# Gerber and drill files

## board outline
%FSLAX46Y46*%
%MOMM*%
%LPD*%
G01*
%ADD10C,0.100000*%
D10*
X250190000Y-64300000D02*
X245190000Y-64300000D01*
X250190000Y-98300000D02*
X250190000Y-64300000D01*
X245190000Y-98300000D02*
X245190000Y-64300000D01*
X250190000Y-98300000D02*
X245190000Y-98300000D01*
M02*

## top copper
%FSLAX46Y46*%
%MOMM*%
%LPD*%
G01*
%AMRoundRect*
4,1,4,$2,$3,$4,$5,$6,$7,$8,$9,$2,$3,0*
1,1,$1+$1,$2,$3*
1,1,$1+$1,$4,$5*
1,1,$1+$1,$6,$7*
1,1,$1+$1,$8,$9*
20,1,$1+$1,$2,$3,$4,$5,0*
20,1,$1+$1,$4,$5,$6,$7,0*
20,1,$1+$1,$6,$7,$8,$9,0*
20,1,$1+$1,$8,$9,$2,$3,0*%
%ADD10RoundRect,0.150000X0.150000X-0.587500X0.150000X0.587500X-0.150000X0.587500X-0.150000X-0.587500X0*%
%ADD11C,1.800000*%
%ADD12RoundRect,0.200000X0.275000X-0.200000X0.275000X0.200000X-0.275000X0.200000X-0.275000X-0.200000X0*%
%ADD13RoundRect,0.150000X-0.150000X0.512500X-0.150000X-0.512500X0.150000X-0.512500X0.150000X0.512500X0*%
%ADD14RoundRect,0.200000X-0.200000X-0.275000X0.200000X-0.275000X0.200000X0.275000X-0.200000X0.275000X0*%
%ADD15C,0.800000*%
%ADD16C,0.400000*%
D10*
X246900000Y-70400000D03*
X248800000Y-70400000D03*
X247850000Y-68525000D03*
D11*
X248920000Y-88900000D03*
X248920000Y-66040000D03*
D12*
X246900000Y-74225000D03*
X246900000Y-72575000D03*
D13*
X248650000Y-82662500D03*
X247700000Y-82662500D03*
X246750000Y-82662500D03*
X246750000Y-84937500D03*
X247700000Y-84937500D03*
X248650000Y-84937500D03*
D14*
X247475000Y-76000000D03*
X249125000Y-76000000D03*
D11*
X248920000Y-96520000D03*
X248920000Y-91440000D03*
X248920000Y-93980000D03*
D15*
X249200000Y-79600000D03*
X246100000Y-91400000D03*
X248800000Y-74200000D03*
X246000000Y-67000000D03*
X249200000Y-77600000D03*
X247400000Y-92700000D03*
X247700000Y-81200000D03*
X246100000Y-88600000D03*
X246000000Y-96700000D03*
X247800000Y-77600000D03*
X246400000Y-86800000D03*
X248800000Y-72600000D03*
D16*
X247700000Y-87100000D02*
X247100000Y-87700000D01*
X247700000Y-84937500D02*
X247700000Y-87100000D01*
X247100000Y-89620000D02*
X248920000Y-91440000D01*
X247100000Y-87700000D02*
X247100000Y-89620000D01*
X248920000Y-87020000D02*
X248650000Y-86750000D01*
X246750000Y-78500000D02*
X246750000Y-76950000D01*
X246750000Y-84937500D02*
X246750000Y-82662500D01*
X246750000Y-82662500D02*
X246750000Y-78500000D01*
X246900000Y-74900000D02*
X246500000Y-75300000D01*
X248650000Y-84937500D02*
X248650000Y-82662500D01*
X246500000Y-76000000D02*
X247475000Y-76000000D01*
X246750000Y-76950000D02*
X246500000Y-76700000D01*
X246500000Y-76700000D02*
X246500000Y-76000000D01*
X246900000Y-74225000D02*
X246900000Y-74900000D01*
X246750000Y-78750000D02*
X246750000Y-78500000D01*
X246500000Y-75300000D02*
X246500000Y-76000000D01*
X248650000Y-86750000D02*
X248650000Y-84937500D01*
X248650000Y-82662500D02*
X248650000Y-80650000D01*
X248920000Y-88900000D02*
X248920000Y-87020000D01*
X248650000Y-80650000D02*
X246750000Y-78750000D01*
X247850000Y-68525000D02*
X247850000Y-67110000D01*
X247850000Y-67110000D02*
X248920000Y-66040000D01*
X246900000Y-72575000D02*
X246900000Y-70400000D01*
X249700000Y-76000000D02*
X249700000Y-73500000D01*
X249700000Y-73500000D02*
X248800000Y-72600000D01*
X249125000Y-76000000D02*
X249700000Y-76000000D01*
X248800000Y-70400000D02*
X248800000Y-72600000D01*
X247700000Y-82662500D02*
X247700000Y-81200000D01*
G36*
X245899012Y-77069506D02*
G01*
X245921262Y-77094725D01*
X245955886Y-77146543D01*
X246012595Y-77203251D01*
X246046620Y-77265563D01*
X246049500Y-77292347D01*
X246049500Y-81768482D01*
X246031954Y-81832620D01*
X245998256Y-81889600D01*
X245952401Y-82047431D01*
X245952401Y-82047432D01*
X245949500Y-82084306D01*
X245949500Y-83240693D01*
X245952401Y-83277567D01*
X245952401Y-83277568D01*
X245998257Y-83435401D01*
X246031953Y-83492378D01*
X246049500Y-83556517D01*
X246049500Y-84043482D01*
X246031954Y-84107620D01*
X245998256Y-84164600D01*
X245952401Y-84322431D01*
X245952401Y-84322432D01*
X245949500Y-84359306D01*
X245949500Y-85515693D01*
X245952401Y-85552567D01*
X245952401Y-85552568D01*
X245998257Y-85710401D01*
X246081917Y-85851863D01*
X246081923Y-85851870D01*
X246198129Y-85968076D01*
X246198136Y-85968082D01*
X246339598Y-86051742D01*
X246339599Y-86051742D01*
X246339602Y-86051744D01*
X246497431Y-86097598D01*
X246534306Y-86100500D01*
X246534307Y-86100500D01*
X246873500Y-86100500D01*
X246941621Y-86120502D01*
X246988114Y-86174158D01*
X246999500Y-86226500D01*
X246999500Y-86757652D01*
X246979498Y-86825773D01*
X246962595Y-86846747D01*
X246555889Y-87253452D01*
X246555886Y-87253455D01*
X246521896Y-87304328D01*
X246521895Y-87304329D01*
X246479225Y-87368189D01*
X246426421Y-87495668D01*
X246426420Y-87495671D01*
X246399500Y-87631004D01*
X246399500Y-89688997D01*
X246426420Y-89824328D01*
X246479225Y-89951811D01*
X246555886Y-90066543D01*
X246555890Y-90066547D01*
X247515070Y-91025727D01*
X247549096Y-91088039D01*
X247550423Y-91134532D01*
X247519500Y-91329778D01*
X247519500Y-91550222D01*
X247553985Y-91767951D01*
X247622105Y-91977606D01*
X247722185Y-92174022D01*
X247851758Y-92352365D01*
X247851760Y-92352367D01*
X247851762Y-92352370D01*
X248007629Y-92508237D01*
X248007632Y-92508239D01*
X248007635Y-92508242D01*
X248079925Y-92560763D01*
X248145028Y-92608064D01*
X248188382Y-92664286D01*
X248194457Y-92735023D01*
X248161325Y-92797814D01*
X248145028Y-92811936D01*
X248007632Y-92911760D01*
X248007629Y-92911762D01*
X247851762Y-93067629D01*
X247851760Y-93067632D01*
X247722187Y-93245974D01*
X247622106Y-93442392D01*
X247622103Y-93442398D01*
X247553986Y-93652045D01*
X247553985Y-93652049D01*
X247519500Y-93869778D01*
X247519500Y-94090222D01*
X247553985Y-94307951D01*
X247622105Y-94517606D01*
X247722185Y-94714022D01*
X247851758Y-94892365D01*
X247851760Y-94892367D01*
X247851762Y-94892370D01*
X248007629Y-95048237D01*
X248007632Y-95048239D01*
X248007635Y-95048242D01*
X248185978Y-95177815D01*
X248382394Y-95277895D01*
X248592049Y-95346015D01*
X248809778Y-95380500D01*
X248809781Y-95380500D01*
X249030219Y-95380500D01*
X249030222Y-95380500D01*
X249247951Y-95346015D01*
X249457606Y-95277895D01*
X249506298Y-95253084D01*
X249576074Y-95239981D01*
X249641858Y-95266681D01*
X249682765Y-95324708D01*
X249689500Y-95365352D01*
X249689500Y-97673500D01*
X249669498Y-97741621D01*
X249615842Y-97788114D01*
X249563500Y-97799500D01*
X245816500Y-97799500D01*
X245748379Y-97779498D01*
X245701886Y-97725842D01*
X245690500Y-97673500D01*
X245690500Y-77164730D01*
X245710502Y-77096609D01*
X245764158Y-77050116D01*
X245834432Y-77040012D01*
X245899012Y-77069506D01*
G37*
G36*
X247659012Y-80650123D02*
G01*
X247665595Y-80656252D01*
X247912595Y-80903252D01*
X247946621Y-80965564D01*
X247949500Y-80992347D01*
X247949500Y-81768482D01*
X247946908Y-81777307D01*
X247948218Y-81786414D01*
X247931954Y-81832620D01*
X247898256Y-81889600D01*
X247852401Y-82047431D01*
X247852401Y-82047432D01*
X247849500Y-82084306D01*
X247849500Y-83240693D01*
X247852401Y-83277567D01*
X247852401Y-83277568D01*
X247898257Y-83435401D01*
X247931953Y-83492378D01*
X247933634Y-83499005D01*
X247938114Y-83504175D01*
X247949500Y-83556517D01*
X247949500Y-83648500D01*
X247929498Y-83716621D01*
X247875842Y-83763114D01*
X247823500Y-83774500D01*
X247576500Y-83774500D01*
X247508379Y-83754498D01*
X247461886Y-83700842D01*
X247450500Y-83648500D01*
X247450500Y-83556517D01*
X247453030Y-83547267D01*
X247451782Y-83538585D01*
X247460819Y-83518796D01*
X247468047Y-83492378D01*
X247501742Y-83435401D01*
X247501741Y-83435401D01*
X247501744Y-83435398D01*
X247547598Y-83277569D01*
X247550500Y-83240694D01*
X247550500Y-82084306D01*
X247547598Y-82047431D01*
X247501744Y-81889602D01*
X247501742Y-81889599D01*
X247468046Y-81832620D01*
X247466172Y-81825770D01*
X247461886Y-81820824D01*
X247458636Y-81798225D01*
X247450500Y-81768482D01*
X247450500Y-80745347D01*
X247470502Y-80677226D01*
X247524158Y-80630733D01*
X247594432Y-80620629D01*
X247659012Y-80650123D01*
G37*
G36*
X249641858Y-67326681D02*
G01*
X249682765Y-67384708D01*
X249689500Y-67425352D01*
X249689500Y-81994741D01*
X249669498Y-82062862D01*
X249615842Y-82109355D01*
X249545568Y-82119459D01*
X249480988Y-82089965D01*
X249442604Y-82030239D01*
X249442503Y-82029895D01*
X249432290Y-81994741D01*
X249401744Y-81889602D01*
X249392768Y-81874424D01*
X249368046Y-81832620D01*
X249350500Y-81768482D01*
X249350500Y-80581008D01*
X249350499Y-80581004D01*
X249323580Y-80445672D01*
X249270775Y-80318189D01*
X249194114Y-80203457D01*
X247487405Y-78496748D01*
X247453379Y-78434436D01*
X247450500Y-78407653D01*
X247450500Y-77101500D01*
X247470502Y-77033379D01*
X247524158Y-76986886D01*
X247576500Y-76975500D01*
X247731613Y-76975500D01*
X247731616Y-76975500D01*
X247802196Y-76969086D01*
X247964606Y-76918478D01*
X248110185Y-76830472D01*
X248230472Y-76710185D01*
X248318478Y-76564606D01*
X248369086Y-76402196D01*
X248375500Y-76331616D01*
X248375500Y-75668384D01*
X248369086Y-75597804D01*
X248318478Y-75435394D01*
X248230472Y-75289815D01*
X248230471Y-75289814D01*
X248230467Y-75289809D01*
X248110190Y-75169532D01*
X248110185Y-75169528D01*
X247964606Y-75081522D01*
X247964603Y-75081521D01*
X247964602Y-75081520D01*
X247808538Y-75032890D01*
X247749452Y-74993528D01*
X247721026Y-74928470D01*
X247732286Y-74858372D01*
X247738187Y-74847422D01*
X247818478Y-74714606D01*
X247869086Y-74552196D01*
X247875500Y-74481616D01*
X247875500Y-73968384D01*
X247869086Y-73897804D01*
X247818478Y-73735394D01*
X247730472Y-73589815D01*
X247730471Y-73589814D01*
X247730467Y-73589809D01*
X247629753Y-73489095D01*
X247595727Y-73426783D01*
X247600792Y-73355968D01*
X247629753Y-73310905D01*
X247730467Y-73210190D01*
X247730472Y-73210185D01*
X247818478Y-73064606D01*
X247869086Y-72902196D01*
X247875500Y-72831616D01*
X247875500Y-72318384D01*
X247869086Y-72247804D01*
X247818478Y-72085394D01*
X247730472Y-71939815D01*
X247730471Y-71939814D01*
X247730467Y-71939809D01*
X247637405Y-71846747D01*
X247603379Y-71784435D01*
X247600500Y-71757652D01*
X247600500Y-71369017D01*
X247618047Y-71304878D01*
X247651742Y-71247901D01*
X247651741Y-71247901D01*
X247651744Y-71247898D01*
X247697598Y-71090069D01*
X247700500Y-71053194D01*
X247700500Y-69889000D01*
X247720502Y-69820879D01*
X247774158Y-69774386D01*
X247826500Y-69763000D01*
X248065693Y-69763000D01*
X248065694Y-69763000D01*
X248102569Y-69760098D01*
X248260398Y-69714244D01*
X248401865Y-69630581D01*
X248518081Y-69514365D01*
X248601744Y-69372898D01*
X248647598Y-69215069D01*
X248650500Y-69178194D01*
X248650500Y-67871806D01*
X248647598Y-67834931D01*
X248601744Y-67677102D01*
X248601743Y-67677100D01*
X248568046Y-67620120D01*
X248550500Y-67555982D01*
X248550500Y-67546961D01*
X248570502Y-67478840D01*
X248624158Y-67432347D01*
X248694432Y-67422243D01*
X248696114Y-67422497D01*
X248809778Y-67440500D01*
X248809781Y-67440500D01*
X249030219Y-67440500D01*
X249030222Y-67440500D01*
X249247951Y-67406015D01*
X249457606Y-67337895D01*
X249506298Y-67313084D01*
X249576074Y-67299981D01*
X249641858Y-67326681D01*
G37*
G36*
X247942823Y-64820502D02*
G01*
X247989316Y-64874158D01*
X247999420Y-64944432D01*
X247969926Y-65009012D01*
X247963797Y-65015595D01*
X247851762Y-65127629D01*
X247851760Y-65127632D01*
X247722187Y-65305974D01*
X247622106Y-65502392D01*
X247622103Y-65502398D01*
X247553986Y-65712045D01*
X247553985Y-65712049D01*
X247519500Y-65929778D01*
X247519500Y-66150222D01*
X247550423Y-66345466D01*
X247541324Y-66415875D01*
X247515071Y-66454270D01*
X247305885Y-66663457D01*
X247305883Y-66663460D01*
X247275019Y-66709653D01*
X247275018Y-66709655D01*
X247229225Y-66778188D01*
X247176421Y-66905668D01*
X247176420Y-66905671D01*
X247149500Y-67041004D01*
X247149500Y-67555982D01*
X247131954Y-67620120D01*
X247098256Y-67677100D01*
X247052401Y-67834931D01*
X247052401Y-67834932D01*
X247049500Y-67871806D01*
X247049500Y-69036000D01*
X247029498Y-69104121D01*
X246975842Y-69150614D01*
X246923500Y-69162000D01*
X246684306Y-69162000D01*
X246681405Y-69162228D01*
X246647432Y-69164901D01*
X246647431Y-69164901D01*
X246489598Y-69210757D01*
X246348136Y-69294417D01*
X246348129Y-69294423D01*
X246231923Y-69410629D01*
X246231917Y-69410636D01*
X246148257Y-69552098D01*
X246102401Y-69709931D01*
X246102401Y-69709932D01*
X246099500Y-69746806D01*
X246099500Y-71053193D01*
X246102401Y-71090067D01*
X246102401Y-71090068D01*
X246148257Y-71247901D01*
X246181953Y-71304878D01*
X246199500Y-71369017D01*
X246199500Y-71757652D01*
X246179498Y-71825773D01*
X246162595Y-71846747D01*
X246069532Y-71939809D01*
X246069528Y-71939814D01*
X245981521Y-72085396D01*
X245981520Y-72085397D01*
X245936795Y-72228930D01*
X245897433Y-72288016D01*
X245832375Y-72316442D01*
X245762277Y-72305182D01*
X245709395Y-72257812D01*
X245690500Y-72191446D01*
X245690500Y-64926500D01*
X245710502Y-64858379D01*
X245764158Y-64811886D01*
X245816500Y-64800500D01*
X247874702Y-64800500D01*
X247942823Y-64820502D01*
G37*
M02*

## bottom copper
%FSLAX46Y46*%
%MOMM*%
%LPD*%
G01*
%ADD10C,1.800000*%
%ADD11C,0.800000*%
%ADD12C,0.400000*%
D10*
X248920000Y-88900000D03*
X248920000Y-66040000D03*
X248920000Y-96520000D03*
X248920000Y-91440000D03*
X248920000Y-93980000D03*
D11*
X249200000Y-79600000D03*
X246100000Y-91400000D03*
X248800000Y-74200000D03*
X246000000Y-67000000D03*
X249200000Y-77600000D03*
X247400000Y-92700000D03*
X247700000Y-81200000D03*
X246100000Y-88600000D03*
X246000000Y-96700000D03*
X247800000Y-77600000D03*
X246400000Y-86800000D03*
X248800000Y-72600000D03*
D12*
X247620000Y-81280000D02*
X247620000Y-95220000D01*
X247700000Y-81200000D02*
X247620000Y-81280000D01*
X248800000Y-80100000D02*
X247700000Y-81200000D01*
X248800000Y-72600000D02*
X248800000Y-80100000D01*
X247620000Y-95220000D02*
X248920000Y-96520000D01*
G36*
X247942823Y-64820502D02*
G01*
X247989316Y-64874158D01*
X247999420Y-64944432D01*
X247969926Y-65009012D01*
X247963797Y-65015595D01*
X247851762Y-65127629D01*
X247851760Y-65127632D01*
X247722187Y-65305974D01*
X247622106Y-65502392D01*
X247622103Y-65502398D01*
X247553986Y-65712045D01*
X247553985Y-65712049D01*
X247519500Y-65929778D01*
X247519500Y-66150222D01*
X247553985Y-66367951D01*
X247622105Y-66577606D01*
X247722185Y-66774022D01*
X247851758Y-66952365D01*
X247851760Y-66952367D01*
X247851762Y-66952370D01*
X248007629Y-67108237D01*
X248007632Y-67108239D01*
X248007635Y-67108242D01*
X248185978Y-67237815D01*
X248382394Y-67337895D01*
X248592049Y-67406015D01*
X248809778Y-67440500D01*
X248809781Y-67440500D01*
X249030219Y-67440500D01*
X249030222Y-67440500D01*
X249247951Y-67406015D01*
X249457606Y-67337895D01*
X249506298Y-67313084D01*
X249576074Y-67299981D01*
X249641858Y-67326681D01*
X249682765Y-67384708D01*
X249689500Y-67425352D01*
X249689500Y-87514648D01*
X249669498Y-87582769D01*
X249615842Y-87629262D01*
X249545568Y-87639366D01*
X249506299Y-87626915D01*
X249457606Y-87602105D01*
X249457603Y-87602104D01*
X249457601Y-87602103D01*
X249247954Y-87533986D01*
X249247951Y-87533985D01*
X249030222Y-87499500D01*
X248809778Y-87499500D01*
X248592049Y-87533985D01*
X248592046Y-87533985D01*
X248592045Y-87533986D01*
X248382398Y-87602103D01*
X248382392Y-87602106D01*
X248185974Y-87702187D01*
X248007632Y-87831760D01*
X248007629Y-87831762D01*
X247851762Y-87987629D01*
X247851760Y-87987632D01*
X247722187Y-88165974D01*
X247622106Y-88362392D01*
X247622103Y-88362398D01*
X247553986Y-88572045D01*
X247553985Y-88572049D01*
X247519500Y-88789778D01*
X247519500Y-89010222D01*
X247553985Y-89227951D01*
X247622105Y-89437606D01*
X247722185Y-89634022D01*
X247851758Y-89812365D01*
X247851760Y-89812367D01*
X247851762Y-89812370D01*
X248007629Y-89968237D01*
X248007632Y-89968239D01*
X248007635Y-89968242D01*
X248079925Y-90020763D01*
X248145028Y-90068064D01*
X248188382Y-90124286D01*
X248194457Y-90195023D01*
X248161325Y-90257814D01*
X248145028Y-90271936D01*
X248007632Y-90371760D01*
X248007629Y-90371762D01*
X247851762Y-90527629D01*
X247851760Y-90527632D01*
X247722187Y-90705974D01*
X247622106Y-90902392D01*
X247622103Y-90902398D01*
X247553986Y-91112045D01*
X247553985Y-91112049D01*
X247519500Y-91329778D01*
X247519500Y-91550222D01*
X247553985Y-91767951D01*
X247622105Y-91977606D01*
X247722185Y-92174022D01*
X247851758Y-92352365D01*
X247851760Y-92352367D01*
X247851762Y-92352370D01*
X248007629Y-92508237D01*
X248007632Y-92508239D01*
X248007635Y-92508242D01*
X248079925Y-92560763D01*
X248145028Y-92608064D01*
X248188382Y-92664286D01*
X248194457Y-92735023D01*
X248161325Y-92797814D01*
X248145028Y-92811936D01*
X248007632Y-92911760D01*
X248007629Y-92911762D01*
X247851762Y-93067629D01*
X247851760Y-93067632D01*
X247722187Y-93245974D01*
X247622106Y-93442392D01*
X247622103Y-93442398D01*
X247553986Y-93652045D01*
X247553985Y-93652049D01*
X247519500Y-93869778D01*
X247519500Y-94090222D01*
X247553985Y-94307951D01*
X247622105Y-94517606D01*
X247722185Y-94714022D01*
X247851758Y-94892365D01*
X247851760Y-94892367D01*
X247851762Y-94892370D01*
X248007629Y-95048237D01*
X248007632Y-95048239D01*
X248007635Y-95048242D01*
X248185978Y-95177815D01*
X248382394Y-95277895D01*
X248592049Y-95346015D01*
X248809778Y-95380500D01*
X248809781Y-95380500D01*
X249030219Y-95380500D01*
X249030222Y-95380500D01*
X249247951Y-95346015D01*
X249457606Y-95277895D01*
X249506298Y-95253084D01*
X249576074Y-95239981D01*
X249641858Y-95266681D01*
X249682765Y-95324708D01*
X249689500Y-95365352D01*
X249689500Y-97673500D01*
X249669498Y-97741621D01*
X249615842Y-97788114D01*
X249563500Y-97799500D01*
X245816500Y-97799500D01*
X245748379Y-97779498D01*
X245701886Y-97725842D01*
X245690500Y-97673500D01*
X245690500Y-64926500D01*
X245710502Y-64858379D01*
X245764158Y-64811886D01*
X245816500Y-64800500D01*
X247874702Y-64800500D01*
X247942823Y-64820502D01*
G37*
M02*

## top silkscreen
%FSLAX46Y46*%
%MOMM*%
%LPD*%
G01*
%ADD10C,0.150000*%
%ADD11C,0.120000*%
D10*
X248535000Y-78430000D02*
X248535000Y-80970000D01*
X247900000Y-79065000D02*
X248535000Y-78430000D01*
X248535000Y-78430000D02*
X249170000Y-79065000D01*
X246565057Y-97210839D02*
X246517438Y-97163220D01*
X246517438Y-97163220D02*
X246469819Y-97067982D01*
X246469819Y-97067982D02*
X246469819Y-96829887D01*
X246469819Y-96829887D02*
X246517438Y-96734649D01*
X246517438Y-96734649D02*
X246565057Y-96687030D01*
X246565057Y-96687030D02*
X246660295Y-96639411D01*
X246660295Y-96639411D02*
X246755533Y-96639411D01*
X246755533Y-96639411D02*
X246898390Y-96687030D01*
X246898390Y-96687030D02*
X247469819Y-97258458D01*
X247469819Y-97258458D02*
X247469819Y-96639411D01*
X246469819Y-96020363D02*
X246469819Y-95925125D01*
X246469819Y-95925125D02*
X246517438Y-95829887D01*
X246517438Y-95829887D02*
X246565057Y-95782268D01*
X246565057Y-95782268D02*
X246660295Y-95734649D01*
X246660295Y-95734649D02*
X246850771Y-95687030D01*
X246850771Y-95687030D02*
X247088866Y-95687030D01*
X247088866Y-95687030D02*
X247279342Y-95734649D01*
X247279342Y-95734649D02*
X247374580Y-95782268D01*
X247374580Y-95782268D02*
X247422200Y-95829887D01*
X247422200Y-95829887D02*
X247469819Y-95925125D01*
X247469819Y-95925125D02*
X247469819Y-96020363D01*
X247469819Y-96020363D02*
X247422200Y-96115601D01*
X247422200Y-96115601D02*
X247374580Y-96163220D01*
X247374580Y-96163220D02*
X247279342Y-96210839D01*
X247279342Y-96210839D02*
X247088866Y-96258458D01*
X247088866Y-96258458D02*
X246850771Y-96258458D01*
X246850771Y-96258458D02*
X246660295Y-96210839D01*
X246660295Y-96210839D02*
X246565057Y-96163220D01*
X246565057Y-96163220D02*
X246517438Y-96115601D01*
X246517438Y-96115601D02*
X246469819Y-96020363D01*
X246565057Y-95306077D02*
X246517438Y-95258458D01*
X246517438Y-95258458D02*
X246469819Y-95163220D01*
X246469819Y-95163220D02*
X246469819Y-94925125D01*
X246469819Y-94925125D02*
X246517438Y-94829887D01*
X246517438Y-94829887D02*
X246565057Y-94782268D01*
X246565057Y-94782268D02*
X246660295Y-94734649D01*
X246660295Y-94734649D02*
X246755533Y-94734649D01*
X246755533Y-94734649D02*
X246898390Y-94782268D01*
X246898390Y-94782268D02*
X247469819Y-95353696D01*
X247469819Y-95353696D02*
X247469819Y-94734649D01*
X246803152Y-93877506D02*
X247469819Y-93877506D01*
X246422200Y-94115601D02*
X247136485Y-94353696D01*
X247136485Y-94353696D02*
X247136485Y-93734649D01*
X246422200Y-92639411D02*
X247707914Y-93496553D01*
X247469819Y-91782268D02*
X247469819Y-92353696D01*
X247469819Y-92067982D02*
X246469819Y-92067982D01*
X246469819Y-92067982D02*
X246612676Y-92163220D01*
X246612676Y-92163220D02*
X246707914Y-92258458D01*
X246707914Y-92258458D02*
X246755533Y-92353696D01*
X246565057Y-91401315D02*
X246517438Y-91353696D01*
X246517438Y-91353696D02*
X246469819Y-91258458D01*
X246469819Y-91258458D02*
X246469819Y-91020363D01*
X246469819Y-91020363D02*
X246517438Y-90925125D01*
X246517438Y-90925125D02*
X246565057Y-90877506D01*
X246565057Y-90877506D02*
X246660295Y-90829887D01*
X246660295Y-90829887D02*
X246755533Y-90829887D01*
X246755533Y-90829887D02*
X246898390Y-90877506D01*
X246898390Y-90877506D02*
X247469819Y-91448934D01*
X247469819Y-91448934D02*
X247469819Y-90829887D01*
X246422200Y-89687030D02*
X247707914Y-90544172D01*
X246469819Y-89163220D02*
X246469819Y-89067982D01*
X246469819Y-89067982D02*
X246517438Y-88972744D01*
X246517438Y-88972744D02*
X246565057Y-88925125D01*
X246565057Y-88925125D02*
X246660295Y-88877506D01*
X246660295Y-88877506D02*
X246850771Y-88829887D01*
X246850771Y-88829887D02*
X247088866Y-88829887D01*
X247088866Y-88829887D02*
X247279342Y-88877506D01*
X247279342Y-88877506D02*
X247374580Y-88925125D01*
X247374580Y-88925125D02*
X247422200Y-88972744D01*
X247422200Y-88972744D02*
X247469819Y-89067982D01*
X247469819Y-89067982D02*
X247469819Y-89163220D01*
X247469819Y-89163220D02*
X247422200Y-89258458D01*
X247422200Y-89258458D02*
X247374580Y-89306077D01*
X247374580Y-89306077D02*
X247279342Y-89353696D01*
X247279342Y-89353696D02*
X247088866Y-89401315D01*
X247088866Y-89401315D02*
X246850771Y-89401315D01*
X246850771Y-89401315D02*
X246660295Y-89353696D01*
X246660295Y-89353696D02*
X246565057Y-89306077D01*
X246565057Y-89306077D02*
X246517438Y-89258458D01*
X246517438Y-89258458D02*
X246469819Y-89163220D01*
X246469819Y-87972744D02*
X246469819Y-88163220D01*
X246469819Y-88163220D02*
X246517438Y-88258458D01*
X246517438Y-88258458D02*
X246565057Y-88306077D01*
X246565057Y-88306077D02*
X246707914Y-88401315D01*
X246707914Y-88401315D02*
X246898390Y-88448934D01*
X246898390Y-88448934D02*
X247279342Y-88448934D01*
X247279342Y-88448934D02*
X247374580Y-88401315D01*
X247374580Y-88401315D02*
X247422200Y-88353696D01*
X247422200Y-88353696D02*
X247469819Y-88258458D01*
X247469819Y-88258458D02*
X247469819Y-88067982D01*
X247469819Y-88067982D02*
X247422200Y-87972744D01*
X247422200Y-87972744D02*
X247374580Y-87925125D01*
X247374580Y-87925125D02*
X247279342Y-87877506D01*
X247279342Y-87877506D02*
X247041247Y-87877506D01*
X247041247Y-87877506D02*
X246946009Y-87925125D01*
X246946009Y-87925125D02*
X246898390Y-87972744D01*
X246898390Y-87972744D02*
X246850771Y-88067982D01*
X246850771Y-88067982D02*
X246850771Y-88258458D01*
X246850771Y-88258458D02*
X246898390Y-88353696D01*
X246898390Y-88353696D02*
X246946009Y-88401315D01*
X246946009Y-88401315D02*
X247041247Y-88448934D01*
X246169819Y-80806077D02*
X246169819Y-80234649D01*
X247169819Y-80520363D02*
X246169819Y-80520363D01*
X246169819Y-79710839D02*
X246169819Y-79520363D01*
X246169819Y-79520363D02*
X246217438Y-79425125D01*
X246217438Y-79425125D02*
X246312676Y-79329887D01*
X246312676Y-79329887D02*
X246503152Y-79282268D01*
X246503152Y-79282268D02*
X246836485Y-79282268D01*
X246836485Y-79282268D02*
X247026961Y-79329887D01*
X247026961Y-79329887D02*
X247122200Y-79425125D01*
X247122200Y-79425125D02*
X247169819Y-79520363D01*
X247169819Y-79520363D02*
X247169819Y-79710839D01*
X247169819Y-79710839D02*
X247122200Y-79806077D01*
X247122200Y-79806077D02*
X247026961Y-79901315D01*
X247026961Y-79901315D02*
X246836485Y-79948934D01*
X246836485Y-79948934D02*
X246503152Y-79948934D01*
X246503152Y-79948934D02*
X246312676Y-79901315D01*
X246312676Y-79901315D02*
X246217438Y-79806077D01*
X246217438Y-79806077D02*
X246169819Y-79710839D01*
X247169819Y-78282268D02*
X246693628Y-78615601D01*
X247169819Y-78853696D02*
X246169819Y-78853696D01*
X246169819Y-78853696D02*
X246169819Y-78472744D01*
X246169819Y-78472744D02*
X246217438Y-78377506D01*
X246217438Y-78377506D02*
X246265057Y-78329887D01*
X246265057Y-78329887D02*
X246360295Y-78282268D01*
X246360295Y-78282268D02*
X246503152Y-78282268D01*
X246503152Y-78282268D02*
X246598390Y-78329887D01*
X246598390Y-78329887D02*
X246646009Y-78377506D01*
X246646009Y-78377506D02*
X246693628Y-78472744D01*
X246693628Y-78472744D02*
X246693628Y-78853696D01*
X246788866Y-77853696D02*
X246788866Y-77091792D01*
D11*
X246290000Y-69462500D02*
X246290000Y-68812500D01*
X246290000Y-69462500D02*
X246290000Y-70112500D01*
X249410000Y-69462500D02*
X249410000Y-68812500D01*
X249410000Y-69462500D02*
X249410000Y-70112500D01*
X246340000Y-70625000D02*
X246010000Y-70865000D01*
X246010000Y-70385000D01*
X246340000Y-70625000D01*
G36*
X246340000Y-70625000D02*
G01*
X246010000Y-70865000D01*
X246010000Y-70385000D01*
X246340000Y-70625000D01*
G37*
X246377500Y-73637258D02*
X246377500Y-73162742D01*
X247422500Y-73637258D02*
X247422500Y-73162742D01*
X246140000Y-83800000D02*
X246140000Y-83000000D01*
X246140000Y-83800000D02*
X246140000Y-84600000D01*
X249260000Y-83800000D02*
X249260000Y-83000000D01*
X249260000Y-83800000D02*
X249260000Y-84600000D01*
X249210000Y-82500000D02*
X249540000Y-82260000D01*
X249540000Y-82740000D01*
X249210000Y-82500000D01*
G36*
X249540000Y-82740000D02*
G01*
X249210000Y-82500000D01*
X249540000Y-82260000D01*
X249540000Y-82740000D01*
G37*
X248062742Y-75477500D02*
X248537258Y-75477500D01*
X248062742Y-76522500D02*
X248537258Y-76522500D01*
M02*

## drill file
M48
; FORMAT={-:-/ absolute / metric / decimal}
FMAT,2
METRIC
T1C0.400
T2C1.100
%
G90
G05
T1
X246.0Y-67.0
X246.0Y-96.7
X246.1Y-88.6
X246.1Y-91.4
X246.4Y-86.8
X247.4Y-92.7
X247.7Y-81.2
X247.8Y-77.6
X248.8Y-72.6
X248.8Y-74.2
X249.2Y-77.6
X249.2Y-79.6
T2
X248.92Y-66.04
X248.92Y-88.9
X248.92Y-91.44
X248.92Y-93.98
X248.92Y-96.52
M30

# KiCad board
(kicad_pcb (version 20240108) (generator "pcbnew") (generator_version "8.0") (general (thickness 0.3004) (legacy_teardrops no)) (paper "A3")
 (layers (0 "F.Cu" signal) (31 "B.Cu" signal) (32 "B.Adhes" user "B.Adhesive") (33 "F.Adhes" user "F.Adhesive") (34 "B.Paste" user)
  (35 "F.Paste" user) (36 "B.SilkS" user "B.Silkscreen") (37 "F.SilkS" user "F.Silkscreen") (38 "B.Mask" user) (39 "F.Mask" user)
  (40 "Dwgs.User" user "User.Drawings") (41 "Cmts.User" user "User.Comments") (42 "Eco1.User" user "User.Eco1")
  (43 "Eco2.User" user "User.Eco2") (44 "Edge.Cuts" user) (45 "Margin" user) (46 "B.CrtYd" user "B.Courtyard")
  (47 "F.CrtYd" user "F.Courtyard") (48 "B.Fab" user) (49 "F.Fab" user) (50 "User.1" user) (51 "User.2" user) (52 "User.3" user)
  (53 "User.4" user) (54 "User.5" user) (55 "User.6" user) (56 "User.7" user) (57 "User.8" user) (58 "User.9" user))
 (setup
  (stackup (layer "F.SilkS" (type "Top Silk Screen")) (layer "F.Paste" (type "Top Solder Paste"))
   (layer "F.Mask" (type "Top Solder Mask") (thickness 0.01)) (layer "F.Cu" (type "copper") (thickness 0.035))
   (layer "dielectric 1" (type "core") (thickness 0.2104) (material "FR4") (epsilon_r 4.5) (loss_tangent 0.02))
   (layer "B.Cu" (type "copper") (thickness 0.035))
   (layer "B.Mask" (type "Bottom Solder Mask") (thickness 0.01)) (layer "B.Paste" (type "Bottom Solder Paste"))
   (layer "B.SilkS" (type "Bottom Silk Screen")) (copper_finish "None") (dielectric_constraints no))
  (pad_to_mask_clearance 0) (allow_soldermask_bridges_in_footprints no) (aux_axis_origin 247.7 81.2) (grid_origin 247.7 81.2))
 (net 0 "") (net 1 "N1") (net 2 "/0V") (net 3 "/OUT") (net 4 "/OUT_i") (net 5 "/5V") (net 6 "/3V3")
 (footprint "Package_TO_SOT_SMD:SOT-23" (layer "F.Cu") (at 247.85 69.4625 90)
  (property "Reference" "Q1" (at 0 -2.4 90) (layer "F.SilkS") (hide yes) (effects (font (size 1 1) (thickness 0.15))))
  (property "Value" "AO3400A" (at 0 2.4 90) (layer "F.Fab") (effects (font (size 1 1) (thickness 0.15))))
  (fp_line (start 0 -1.56) (end 0.65 -1.56) (stroke (width 0.12) (type solid)) (layer "F.SilkS"))
  (fp_line (start 0 -1.56) (end -0.65 -1.56) (stroke (width 0.12) (type solid)) (layer "F.SilkS"))
  (fp_line (start 0 1.56) (end 0.65 1.56) (stroke (width 0.12) (type solid)) (layer "F.SilkS"))
  (fp_line (start 0 1.56) (end -0.65 1.56) (stroke (width 0.12) (type solid)) (layer "F.SilkS"))
  (fp_poly
   (pts (xy -1.1625 -1.51) (xy -1.4025 -1.84) (xy -0.9225 -1.84) (xy -1.1625 -1.51)) (stroke (width 0.12) (type solid)) (fill solid)
   (layer "F.SilkS"))
  (pad "1" smd roundrect (at -0.9375 -0.95 90) (size 1.475 0.6) (layers "F.Cu" "F.Paste" "F.Mask") (roundrect_rratio 0.25) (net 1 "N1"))
  (pad "2" smd roundrect (at -0.9375 0.95 90) (size 1.475 0.6) (layers "F.Cu" "F.Paste" "F.Mask") (roundrect_rratio 0.25) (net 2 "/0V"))
  (pad "3" smd roundrect (at 0.9375 0 90) (size 1.475 0.6) (layers "F.Cu" "F.Paste" "F.Mask") (roundrect_rratio 0.25) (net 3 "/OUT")))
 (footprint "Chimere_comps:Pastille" (layer "F.Cu") (at 248.92 88.9)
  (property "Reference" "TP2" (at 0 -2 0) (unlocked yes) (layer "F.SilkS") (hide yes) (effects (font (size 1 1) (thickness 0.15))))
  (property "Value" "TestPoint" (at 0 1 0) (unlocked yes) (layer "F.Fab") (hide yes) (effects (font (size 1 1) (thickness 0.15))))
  (pad "1" thru_hole circle (at 0 0) (size 1.8 1.8) (drill 1.1) (layers "*.Cu" "*.Mask") (remove_unused_layers no) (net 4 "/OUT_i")))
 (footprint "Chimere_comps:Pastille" (layer "F.Cu") (at 248.92 66.04)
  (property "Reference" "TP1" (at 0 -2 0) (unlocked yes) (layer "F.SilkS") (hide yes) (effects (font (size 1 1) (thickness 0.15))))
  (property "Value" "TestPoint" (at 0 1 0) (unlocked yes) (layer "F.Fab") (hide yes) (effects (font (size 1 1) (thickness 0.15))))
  (pad "1" thru_hole circle (at 0 0) (size 1.8 1.8) (drill 1.1) (layers "*.Cu" "*.Mask") (remove_unused_layers no) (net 3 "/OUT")))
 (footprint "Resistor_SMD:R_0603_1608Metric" (layer "F.Cu") (at 246.9 73.4 90)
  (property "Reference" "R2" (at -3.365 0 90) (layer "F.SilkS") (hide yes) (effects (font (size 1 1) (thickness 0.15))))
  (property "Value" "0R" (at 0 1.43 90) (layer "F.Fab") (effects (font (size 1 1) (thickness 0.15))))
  (fp_line (start -0.237258 -0.5225) (end 0.237258 -0.5225) (stroke (width 0.12) (type solid)) (layer "F.SilkS"))
  (fp_line (start -0.237258 0.5225) (end 0.237258 0.5225) (stroke (width 0.12) (type solid)) (layer "F.SilkS"))
  (pad "1" smd roundrect (at -0.825 0 90) (size 0.8 0.95) (layers "F.Cu" "F.Paste" "F.Mask") (roundrect_rratio 0.25) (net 4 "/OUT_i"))
  (pad "2" smd roundrect (at 0.825 0 90) (size 0.8 0.95) (layers "F.Cu" "F.Paste" "F.Mask") (roundrect_rratio 0.25) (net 1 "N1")))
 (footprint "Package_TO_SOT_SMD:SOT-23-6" (layer "F.Cu") (at 247.7 83.8 -90)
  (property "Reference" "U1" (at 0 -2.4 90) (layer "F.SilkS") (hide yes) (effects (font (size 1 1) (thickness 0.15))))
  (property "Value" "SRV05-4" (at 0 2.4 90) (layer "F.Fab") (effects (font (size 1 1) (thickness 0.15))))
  (fp_line (start 0 1.56) (end -0.8 1.56) (stroke (width 0.12) (type solid)) (layer "F.SilkS"))
  (fp_line (start 0 1.56) (end 0.8 1.56) (stroke (width 0.12) (type solid)) (layer "F.SilkS"))
  (fp_line (start 0 -1.56) (end -0.8 -1.56) (stroke (width 0.12) (type solid)) (layer "F.SilkS"))
  (fp_line (start 0 -1.56) (end 0.8 -1.56) (stroke (width 0.12) (type solid)) (layer "F.SilkS"))
  (fp_poly
   (pts (xy -1.3 -1.51) (xy -1.54 -1.84) (xy -1.06 -1.84) (xy -1.3 -1.51)) (stroke (width 0.12) (type solid)) (fill solid) (layer "F.SilkS"))
  (pad "1" smd roundrect (at -1.1375 -0.95 270) (size 1.325 0.6) (layers "F.Cu" "F.Paste" "F.Mask") (roundrect_rratio 0.25) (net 4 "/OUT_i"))
  (pad "2" smd roundrect (at -1.1375 0 270) (size 1.325 0.6) (layers "F.Cu" "F.Paste" "F.Mask") (roundrect_rratio 0.25) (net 2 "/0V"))
  (pad "3" smd roundrect (at -1.1375 0.95 270) (size 1.325 0.6) (layers "F.Cu" "F.Paste" "F.Mask") (roundrect_rratio 0.25) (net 4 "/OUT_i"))
  (pad "4" smd roundrect (at 1.1375 0.95 270) (size 1.325 0.6) (layers "F.Cu" "F.Paste" "F.Mask") (roundrect_rratio 0.25) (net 4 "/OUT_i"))
  (pad "5" smd roundrect (at 1.1375 0 270) (size 1.325 0.6) (layers "F.Cu" "F.Paste" "F.Mask") (roundrect_rratio 0.25) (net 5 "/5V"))
  (pad "6" smd roundrect (at 1.1375 -0.95 270) (size 1.325 0.6) (layers "F.Cu" "F.Paste" "F.Mask") (roundrect_rratio 0.25) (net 4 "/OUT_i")))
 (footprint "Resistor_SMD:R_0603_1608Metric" (layer "F.Cu") (at 248.3 76)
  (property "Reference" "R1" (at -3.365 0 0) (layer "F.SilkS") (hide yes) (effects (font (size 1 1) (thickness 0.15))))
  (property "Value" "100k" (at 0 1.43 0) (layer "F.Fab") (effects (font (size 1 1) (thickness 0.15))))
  (fp_line (start -0.237258 -0.5225) (end 0.237258 -0.5225) (stroke (width 0.12) (type solid)) (layer "F.SilkS"))
  (fp_line (start -0.237258 0.5225) (end 0.237258 0.5225) (stroke (width 0.12) (type solid)) (layer "F.SilkS"))
  (pad "1" smd roundrect (at -0.825 0) (size 0.8 0.95) (layers "F.Cu" "F.Paste" "F.Mask") (roundrect_rratio 0.25) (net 4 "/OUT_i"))
  (pad "2" smd roundrect (at 0.825 0) (size 0.8 0.95) (layers "F.Cu" "F.Paste" "F.Mask") (roundrect_rratio 0.25) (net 2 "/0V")))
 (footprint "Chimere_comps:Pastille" (layer "F.Cu") (at 248.92 96.52)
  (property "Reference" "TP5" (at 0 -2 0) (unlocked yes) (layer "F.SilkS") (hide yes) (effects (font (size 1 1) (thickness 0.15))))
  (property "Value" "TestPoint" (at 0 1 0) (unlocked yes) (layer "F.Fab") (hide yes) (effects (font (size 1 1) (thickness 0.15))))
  (pad "1" thru_hole circle (at 0 0) (size 1.8 1.8) (drill 1.1) (layers "*.Cu" "*.Mask") (remove_unused_layers no) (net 2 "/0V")))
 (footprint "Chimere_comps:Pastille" (layer "F.Cu") (at 248.92 91.44)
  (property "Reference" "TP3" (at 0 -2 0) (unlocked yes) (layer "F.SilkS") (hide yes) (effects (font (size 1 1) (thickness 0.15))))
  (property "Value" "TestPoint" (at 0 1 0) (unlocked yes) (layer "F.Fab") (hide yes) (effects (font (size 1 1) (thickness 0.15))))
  (pad "1" thru_hole circle (at 0 0) (size 1.8 1.8) (drill 1.1) (layers "*.Cu" "*.Mask") (remove_unused_layers no) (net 5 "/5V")))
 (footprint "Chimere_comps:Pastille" (layer "F.Cu") (at 248.92 93.98)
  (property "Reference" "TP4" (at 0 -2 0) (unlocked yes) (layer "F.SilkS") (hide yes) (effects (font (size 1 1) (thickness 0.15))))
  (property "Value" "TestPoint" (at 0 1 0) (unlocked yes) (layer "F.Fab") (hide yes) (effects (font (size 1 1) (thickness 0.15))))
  (pad "1" thru_hole circle (at 0 0) (size 1.8 1.8) (drill 1.1) (layers "*.Cu" "*.Mask") (remove_unused_layers no) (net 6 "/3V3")))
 (gr_line (start 248.535 78.43) (end 248.535 80.97) (stroke (width 0.15) (type solid)) (layer "F.SilkS"))
 (gr_line (start 247.9 79.065) (end 248.535 78.43) (stroke (width 0.15) (type solid)) (layer "F.SilkS"))
 (gr_line (start 248.535 78.43) (end 249.17 79.065) (stroke (width 0.15) (type solid)) (layer "F.SilkS"))
 (gr_line (start 250.19 64.3) (end 245.19 64.3) (stroke (width 0.1) (type default)) (layer "Edge.Cuts"))
 (gr_line (start 250.19 98.3) (end 250.19 64.3) (stroke (width 0.1) (type default)) (layer "Edge.Cuts"))
 (gr_line (start 245.19 98.3) (end 245.19 64.3) (stroke (width 0.1) (type default)) (layer "Edge.Cuts"))
 (gr_line (start 250.19 98.3) (end 245.19 98.3) (stroke (width 0.1) (type default)) (layer "Edge.Cuts"))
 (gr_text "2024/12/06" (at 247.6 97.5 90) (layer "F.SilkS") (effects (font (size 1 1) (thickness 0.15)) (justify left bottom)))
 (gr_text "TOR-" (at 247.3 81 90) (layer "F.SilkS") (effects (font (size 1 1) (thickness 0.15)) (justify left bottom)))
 (segment (start 247.7 87.1) (end 247.1 87.7) (width 0.4) (layer "F.Cu") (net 5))
 (segment (start 247.7 84.9375) (end 247.7 87.1) (width 0.4) (layer "F.Cu") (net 5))
 (segment (start 247.1 89.62) (end 248.92 91.44) (width 0.4) (layer "F.Cu") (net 5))
 (segment (start 247.1 87.7) (end 247.1 89.62) (width 0.4) (layer "F.Cu") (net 5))
 (segment (start 248.92 87.02) (end 248.65 86.75) (width 0.4) (layer "F.Cu") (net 4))
 (segment (start 246.75 78.5) (end 246.75 76.95) (width 0.4) (layer "F.Cu") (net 4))
 (segment (start 246.75 84.9375) (end 246.75 82.6625) (width 0.4) (layer "F.Cu") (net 4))
 (segment (start 246.75 82.6625) (end 246.75 78.5) (width 0.4) (layer "F.Cu") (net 4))
 (segment (start 246.9 74.9) (end 246.5 75.3) (width 0.4) (layer "F.Cu") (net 4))
 (segment (start 248.65 84.9375) (end 248.65 82.6625) (width 0.4) (layer "F.Cu") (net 4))
 (segment (start 246.5 76) (end 247.475 76) (width 0.4) (layer "F.Cu") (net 4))
 (segment (start 246.75 76.95) (end 246.5 76.7) (width 0.4) (layer "F.Cu") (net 4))
 (segment (start 246.5 76.7) (end 246.5 76) (width 0.4) (layer "F.Cu") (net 4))
 (segment (start 246.9 74.225) (end 246.9 74.9) (width 0.4) (layer "F.Cu") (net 4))
 (segment (start 246.75 78.75) (end 246.75 78.5) (width 0.4) (layer "F.Cu") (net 4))
 (segment (start 246.5 75.3) (end 246.5 76) (width 0.4) (layer "F.Cu") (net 4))
 (segment (start 248.65 86.75) (end 248.65 84.9375) (width 0.4) (layer "F.Cu") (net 4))
 (segment (start 248.65 82.6625) (end 248.65 80.65) (width 0.4) (layer "F.Cu") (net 4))
 (segment (start 248.92 88.9) (end 248.92 87.02) (width 0.4) (layer "F.Cu") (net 4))
 (segment (start 248.65 80.65) (end 246.75 78.75) (width 0.4) (layer "F.Cu") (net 4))
 (segment (start 247.85 68.525) (end 247.85 67.11) (width 0.4) (layer "F.Cu") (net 3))
 (segment (start 247.85 67.11) (end 248.92 66.04) (width 0.4) (layer "F.Cu") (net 3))
 (segment (start 246.9 72.575) (end 246.9 70.4) (width 0.4) (layer "F.Cu") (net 1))
 (segment (start 249.7 76) (end 249.7 73.5) (width 0.4) (layer "F.Cu") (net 2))
 (segment (start 249.7 73.5) (end 248.8 72.6) (width 0.4) (layer "F.Cu") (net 2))
 (segment (start 249.125 76) (end 249.7 76) (width 0.4) (layer "F.Cu") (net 2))
 (segment (start 248.8 70.4) (end 248.8 72.6) (width 0.4) (layer "F.Cu") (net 2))
 (segment (start 247.7 82.6625) (end 247.7 81.2) (width 0.4) (layer "F.Cu") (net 2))
 (via (at 249.2 79.6) (size 0.8) (drill 0.4) (layers "F.Cu" "B.Cu") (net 2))
 (via (at 246.1 91.4) (size 0.8) (drill 0.4) (layers "F.Cu" "B.Cu") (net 2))
 (via (at 248.8 74.2) (size 0.8) (drill 0.4) (layers "F.Cu" "B.Cu") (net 2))
 (via (at 246 67) (size 0.8) (drill 0.4) (layers "F.Cu" "B.Cu") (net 2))
 (via (at 249.2 77.6) (size 0.8) (drill 0.4) (layers "F.Cu" "B.Cu") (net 2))
 (via (at 247.4 92.7) (size 0.8) (drill 0.4) (layers "F.Cu" "B.Cu") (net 2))
 (via (at 247.7 81.2) (size 0.8) (drill 0.4) (layers "F.Cu" "B.Cu") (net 2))
 (via (at 246.1 88.6) (size 0.8) (drill 0.4) (layers "F.Cu" "B.Cu") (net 2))
 (via (at 246 96.7) (size 0.8) (drill 0.4) (layers "F.Cu" "B.Cu") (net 2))
 (via (at 247.8 77.6) (size 0.8) (drill 0.4) (layers "F.Cu" "B.Cu") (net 2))
 (via (at 246.4 86.8) (size 0.8) (drill 0.4) (layers "F.Cu" "B.Cu") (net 2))
 (via (at 248.8 72.6) (size 0.8) (drill 0.4) (layers "F.Cu" "B.Cu") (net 2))
 (segment (start 247.62 81.28) (end 247.62 95.22) (width 0.4) (layer "B.Cu") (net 2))
 (segment (start 247.7 81.2) (end 247.62 81.28) (width 0.4) (layer "B.Cu") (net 2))
 (segment (start 248.8 80.1) (end 247.7 81.2) (width 0.4) (layer "B.Cu") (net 2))
 (segment (start 248.8 72.6) (end 248.8 80.1) (width 0.4) (layer "B.Cu") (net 2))
 (segment (start 247.62 95.22) (end 248.92 96.52) (width 0.4) (layer "B.Cu") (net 2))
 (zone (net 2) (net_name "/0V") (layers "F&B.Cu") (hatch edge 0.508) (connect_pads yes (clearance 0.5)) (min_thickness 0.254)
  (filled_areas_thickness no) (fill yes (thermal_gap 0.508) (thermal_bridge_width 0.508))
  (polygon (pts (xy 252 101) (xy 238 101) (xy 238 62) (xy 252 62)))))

